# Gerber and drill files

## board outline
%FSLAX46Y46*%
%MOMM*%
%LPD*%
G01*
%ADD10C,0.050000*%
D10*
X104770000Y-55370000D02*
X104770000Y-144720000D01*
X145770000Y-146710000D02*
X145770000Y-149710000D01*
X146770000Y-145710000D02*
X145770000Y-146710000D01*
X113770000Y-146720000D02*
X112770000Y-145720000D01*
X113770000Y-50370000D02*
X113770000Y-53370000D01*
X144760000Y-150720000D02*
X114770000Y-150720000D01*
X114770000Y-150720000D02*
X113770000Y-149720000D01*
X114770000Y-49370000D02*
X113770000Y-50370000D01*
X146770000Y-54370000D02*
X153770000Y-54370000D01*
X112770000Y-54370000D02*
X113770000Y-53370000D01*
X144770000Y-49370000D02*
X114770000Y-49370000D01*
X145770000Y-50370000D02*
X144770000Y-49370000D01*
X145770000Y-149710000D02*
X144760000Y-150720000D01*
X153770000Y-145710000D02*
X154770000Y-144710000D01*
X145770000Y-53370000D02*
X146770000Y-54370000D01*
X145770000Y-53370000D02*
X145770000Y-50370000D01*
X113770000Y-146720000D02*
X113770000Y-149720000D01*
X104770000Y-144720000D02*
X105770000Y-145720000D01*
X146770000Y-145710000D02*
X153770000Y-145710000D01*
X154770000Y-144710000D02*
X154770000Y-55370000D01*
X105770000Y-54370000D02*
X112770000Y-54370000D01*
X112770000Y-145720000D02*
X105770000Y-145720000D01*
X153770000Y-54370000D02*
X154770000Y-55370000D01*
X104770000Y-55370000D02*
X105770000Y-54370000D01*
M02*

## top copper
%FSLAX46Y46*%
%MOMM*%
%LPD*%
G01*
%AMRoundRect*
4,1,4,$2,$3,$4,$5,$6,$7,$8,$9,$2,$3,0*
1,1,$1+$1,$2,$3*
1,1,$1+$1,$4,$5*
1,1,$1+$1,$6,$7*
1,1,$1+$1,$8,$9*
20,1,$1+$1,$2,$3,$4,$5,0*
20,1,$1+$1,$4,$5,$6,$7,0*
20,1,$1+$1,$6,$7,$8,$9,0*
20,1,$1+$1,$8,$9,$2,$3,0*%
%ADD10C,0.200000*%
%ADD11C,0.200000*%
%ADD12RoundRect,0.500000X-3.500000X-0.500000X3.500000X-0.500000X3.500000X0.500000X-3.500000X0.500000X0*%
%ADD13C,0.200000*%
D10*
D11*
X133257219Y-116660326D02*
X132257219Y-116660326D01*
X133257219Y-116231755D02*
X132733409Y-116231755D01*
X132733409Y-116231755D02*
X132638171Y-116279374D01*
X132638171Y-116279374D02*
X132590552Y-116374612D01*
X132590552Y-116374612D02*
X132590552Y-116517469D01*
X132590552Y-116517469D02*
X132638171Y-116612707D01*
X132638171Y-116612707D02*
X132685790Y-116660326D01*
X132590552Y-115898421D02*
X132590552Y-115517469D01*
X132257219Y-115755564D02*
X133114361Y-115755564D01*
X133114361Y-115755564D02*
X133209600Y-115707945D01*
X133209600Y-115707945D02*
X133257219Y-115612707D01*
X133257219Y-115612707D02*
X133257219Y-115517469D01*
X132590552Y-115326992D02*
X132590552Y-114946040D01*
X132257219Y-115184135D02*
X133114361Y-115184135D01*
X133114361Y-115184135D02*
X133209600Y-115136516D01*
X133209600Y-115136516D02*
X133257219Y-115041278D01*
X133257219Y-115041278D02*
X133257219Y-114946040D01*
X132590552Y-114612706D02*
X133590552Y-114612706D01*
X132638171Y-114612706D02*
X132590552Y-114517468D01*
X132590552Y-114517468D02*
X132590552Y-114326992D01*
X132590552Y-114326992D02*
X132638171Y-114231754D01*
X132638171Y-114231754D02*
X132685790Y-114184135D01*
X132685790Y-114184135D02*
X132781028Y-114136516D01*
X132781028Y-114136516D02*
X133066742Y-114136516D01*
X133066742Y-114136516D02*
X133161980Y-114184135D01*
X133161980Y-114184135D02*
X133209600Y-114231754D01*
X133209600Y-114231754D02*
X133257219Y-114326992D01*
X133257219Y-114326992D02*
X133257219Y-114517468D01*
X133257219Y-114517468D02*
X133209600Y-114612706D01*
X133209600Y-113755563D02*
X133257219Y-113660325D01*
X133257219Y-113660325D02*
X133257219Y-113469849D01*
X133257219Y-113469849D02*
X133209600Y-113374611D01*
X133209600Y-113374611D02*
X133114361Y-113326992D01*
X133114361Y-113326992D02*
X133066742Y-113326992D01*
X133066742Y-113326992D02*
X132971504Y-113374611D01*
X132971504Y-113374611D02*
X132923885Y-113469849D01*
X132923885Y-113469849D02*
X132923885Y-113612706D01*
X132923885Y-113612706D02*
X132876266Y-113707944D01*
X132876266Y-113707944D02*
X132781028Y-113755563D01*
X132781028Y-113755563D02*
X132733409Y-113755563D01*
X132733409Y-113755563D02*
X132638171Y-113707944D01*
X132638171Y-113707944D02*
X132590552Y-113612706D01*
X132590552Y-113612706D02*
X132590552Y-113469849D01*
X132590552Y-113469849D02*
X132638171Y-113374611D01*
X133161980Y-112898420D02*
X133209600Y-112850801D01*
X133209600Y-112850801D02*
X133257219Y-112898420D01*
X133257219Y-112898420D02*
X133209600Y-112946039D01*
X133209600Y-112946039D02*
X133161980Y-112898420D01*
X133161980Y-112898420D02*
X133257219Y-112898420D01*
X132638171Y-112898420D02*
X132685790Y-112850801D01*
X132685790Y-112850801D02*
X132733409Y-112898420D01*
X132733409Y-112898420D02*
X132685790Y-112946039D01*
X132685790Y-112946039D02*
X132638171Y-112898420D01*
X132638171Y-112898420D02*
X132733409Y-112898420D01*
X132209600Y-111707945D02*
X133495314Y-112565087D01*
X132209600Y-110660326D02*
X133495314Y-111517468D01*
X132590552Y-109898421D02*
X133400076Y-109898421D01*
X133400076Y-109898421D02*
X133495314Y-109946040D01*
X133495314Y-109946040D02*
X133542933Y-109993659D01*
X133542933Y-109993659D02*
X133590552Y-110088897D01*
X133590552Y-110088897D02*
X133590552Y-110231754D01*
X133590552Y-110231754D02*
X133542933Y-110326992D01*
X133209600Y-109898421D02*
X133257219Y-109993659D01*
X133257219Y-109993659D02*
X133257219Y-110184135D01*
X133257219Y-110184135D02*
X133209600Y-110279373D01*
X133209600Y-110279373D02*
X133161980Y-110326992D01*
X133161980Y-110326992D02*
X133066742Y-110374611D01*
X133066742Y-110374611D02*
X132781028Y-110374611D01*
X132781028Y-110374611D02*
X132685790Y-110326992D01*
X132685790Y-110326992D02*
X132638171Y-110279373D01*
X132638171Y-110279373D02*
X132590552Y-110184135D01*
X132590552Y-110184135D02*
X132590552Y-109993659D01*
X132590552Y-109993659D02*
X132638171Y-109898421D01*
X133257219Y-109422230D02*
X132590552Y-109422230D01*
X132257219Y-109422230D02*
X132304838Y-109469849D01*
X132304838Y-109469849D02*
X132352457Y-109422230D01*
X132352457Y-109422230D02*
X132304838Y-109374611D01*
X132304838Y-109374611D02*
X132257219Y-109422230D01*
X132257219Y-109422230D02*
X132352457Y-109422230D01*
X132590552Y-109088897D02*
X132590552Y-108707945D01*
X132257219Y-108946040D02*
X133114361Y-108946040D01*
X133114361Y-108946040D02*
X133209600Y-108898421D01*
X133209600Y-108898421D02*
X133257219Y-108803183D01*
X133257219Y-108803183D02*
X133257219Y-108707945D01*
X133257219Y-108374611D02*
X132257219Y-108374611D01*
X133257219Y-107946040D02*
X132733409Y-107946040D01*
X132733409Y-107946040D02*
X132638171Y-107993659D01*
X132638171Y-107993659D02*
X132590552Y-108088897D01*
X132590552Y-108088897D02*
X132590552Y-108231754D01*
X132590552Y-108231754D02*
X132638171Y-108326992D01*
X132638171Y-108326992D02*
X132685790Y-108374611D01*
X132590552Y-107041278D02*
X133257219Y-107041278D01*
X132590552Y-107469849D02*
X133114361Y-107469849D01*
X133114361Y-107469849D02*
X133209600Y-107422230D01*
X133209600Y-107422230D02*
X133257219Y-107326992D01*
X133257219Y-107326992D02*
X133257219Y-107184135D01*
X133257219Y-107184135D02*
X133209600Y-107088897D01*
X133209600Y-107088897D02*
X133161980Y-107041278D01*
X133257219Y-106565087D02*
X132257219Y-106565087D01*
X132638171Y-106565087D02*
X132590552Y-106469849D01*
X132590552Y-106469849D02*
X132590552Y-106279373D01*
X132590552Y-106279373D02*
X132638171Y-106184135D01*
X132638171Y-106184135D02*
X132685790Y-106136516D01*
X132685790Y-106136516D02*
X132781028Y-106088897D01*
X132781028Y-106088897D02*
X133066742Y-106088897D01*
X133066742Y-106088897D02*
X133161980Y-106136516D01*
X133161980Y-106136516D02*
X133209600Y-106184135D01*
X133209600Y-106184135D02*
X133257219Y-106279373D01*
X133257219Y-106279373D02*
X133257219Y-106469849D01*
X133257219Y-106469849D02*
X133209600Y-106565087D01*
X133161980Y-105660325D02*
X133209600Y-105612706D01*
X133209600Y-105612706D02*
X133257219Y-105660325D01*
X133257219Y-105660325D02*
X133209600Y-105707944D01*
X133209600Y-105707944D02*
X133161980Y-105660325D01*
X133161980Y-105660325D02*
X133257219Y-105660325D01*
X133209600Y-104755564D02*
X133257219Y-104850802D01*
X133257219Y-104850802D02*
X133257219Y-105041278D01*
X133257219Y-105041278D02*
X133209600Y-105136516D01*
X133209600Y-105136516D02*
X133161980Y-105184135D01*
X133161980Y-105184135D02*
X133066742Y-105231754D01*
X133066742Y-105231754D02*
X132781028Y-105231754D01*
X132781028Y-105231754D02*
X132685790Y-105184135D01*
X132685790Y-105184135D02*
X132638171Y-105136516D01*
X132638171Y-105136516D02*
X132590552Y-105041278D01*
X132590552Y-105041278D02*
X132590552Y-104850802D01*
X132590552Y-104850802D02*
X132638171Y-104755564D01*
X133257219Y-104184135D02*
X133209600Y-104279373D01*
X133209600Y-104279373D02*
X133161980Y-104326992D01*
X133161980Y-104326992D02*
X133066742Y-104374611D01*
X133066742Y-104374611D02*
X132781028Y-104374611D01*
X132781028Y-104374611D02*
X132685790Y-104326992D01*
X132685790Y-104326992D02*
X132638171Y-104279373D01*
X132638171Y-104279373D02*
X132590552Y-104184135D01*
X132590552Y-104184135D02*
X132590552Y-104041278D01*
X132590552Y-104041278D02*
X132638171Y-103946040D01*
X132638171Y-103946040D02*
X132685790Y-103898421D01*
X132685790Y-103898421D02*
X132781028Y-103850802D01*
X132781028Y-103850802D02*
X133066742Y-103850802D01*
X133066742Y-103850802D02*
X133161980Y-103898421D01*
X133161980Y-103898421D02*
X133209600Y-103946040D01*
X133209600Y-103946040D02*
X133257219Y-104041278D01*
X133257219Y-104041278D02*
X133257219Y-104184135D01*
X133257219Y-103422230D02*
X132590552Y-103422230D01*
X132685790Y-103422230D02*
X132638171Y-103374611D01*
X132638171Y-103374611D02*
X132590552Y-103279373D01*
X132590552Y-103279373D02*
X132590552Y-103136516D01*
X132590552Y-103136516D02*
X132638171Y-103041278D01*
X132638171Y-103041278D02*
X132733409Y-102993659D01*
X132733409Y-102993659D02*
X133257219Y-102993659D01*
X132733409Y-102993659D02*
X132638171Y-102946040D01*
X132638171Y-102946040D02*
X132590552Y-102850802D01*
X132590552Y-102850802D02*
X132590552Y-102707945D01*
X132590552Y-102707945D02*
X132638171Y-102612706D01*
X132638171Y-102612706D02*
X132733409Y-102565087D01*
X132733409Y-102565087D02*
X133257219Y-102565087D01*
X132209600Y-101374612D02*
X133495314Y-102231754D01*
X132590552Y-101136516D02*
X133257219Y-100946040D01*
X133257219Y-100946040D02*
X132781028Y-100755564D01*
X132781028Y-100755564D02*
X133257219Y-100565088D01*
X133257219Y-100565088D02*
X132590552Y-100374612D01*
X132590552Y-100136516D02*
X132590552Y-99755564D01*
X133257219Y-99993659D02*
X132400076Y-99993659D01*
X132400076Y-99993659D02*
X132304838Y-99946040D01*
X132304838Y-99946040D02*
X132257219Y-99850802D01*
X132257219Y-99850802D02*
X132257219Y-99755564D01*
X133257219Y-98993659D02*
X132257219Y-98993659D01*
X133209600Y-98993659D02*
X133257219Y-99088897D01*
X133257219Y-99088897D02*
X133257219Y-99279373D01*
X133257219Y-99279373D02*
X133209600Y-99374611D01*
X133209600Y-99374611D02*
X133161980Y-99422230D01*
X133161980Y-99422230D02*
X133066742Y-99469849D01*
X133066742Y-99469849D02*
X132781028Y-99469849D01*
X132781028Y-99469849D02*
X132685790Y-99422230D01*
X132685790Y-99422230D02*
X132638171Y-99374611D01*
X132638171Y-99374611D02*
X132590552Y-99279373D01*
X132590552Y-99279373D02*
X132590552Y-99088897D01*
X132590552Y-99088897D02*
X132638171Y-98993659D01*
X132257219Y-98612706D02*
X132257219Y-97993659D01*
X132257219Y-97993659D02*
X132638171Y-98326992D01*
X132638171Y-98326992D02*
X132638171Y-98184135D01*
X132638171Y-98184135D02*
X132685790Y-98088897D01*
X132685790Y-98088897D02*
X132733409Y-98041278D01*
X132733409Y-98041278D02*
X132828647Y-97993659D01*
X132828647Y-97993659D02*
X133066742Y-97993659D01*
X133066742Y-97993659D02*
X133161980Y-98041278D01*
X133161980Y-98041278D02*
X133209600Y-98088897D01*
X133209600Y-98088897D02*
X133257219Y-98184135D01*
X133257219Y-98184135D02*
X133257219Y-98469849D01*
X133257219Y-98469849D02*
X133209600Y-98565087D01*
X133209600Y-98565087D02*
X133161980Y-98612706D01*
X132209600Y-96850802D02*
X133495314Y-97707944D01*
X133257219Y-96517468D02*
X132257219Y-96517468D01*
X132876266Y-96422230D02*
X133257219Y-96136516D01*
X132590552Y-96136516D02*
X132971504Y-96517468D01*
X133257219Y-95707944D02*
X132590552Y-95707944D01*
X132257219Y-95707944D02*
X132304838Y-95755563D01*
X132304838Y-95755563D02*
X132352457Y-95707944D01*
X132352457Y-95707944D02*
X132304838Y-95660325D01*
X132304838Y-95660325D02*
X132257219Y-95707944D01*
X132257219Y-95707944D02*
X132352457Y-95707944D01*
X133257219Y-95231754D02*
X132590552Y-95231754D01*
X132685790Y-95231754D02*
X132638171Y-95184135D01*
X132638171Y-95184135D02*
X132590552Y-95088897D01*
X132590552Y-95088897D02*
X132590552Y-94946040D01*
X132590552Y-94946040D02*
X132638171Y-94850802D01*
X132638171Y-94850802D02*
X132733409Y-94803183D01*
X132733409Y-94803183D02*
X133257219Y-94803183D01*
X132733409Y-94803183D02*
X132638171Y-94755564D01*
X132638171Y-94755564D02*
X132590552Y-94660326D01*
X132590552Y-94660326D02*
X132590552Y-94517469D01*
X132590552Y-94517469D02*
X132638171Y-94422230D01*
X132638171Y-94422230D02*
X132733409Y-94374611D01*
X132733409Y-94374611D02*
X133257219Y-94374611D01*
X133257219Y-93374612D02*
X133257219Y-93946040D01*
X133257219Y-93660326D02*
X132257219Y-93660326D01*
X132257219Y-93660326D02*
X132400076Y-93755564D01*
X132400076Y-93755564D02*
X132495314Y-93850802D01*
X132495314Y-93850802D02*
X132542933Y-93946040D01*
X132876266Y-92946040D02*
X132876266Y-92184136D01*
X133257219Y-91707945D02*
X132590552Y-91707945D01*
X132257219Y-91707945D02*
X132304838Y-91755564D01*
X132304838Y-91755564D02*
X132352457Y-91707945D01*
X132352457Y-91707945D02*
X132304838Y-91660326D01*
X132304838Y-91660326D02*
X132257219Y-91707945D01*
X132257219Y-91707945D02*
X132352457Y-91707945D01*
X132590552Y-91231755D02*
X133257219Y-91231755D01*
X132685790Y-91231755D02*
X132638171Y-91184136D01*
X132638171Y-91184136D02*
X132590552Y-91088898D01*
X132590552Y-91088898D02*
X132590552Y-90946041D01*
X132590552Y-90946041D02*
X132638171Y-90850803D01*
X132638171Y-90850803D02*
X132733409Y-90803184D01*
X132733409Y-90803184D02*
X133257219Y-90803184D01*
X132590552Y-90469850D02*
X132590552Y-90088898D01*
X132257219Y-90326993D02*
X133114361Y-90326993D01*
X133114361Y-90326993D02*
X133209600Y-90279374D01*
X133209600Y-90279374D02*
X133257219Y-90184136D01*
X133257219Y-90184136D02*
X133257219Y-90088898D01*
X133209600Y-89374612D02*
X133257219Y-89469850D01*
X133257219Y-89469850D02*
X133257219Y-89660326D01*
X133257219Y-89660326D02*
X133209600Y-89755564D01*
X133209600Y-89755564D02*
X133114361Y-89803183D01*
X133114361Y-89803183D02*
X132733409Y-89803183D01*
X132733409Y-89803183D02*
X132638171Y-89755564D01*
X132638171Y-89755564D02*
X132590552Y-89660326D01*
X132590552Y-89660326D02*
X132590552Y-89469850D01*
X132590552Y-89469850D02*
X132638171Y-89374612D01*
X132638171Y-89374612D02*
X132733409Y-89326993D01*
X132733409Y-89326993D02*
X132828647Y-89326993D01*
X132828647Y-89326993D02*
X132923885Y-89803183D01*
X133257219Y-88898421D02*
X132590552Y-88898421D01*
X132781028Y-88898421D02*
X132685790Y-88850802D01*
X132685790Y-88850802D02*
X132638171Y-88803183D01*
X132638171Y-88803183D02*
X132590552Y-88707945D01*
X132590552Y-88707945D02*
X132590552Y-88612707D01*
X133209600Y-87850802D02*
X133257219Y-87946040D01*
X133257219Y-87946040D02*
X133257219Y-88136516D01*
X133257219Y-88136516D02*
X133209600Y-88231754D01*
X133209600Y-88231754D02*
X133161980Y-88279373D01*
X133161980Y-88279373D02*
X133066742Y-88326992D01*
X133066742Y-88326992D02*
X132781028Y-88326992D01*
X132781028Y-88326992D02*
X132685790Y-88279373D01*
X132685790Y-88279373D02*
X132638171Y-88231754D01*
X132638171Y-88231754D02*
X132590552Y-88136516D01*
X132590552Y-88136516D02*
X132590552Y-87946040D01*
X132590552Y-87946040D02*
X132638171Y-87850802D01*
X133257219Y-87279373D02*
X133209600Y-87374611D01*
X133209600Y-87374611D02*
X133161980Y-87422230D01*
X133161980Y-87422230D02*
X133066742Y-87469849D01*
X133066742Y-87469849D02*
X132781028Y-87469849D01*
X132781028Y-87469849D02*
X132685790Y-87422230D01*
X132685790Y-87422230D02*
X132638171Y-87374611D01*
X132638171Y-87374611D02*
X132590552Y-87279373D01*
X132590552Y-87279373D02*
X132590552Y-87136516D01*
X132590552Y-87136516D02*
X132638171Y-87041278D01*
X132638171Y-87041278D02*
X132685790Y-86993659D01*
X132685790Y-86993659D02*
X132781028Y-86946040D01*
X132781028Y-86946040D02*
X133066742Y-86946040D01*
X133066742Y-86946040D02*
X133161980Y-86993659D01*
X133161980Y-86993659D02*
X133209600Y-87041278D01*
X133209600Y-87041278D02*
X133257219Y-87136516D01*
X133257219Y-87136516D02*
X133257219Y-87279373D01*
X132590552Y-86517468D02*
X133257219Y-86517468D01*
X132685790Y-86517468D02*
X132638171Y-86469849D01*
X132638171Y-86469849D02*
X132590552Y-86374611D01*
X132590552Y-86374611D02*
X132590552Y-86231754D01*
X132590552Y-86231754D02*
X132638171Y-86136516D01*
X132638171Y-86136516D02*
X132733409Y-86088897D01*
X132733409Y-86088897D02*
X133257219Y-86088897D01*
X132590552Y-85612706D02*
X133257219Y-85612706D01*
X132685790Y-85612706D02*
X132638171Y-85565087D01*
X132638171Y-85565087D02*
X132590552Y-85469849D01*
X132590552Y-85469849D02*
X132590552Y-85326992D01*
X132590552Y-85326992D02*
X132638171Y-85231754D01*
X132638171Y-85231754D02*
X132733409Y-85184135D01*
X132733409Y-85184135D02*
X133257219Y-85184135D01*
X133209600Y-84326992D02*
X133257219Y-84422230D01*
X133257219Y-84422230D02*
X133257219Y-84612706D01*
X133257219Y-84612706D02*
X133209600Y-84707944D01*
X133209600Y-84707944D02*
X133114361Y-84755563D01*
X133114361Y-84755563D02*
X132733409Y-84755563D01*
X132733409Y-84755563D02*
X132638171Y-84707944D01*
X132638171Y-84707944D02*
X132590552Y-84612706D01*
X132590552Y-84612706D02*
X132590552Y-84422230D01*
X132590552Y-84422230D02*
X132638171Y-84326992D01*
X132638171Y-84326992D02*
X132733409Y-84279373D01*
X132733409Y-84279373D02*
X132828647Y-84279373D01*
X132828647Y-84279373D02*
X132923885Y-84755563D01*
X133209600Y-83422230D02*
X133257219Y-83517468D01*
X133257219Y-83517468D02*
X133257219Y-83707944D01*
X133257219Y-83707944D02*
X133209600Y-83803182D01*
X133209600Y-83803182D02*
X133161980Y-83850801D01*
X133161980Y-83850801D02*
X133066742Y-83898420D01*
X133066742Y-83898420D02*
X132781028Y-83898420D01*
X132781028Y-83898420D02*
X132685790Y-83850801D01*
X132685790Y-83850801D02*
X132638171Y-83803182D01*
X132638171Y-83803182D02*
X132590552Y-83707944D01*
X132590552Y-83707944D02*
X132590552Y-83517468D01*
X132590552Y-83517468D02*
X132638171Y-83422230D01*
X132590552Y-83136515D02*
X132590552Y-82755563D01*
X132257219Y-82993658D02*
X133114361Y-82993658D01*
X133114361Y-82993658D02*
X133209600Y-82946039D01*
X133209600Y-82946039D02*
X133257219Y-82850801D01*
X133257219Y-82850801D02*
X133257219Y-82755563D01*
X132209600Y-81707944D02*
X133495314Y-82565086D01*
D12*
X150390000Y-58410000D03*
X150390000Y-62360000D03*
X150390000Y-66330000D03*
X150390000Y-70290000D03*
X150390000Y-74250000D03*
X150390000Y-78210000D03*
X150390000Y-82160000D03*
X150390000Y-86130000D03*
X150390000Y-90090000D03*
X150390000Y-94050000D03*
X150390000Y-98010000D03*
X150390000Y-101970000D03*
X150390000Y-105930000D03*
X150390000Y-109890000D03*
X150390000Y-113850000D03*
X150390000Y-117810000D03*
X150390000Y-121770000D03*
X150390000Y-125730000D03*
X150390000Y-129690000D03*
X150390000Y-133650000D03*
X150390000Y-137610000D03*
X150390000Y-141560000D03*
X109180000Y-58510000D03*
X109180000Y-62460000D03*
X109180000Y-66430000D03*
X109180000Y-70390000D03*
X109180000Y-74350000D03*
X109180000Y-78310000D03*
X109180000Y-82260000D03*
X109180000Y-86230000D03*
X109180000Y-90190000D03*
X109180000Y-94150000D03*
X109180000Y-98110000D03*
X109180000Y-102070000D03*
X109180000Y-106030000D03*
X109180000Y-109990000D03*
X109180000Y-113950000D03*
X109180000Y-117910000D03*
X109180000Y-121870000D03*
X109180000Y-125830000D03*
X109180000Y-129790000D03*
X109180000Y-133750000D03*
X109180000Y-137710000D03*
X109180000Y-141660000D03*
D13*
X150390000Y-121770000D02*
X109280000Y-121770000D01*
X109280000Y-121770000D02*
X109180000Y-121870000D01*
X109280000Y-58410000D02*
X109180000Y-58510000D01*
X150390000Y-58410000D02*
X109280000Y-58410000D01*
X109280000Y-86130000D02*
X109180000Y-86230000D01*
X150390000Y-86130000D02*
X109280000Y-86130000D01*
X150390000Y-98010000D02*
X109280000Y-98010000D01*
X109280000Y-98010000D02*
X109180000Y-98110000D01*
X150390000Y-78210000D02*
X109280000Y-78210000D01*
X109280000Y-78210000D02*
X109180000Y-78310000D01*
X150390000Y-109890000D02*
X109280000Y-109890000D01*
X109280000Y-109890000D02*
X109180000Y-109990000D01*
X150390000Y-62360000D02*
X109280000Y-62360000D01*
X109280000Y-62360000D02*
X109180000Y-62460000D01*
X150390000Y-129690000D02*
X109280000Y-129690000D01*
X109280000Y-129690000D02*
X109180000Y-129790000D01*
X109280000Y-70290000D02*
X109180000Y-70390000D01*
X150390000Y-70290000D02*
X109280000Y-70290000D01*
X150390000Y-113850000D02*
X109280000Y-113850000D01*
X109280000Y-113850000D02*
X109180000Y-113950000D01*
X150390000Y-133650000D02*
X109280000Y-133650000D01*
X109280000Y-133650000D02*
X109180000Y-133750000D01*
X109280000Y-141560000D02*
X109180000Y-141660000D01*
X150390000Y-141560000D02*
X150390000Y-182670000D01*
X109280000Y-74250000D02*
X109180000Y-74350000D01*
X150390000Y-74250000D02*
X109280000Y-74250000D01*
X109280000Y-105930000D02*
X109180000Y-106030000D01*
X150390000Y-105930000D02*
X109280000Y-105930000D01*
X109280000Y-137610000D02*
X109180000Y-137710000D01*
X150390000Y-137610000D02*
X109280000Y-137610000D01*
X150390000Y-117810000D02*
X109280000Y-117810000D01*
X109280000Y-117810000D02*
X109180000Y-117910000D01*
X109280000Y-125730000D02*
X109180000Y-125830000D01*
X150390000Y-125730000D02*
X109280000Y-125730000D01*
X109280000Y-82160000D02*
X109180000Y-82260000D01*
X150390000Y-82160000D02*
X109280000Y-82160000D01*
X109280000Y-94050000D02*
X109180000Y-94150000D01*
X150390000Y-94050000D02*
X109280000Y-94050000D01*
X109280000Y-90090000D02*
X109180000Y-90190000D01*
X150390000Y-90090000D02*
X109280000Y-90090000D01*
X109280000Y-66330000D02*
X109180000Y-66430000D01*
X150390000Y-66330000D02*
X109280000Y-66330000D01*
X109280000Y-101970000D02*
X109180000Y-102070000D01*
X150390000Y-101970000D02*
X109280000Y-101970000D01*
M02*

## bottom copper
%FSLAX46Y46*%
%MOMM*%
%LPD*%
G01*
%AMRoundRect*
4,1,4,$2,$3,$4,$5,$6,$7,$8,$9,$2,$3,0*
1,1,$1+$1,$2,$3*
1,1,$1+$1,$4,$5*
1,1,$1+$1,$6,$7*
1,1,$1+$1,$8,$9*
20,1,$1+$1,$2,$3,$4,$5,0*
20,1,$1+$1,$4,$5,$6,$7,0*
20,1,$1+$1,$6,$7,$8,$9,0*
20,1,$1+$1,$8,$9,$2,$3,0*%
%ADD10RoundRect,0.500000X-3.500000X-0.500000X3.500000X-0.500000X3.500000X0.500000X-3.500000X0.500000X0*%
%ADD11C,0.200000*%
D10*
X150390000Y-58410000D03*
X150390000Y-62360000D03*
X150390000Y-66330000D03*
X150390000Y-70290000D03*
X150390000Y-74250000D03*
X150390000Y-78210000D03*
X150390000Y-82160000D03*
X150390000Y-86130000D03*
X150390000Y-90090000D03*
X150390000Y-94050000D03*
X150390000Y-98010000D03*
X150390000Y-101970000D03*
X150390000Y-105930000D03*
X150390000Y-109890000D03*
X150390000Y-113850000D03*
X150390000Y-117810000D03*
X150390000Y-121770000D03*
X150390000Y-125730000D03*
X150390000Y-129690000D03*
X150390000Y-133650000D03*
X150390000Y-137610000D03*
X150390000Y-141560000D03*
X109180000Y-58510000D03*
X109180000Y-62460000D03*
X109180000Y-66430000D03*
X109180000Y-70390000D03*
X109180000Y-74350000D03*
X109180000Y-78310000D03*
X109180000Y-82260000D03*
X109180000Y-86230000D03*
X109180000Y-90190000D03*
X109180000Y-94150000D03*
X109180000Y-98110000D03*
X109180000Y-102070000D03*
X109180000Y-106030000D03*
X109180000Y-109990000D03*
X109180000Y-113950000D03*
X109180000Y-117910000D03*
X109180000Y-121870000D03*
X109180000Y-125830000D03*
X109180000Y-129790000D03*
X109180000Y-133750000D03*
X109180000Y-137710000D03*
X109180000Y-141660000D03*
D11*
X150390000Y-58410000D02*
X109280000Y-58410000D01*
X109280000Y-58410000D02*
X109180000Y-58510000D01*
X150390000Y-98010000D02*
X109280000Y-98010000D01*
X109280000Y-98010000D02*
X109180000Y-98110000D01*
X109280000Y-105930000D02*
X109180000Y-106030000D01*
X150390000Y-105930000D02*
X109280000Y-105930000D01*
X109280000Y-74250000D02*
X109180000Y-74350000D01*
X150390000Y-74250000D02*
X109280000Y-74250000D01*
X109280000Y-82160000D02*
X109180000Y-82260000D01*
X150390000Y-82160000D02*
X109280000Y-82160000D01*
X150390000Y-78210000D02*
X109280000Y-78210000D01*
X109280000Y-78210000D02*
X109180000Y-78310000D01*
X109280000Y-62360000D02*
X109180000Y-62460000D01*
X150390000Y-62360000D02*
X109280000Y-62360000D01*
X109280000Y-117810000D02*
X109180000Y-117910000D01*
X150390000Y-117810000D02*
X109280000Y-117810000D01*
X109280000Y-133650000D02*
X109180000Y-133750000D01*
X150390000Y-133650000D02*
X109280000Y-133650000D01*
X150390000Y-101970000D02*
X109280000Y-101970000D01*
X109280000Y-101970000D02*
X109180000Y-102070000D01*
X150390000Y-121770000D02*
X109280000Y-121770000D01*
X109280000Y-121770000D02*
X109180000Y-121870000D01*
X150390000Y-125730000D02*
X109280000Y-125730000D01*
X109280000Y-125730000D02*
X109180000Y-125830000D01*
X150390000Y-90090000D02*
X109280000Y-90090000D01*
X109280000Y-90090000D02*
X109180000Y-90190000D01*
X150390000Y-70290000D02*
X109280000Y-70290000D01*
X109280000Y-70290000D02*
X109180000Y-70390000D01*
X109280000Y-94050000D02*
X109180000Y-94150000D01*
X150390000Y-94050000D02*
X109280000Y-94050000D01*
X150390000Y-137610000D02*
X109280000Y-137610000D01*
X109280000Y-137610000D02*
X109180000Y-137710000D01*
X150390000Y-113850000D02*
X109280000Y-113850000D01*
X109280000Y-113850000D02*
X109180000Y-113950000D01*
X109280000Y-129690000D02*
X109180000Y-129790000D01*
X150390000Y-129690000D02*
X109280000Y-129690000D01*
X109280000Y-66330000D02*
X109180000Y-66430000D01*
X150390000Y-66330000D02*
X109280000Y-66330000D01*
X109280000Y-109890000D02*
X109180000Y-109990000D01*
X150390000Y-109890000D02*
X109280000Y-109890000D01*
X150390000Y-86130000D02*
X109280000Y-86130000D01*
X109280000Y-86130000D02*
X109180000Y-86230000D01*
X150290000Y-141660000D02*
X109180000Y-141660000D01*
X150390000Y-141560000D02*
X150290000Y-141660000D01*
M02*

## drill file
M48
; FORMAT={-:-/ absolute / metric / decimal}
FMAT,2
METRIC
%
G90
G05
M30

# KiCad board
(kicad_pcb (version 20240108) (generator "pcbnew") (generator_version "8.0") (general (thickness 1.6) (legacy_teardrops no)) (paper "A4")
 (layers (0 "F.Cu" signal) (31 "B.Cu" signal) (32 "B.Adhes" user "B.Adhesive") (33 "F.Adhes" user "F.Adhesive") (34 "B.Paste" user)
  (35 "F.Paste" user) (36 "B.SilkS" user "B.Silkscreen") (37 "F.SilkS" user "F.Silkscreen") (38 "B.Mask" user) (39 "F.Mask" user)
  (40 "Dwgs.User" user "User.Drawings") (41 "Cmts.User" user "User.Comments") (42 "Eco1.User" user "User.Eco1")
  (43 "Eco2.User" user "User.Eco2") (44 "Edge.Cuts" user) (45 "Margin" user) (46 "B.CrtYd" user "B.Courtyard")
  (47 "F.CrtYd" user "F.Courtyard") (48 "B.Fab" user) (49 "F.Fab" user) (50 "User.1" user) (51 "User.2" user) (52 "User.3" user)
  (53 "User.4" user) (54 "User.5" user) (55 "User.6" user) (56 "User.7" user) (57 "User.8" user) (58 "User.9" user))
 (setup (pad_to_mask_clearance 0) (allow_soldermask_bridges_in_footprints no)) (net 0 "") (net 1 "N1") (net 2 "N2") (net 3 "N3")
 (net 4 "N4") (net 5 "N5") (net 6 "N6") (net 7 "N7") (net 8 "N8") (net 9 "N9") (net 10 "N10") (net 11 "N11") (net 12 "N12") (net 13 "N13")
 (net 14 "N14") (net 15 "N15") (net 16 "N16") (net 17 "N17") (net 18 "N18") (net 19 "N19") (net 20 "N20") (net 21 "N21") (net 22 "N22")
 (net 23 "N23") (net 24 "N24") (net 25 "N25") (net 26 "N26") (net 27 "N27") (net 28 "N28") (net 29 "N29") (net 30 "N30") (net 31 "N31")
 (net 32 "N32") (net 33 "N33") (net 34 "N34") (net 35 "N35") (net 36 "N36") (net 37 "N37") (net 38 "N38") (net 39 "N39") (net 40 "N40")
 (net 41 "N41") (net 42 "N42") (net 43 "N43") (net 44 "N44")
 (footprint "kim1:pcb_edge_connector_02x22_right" (layer "F.Cu") (at 145.04 98.96)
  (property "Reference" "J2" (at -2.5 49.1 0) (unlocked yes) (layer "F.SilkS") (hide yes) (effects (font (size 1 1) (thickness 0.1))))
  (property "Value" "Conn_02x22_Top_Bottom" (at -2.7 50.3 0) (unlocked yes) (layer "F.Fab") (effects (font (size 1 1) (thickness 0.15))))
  (pad "1" connect roundrect (at 5.35 -40.55) (size 8 2) (layers "F.Cu" "F.Mask") (roundrect_rratio 0.25) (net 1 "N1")
   (thermal_bridge_angle 45))
  (pad "2" connect roundrect (at 5.35 -36.6) (size 8 2) (layers "F.Cu" "F.Mask") (roundrect_rratio 0.25) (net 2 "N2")
   (thermal_bridge_angle 45))
  (pad "3" connect roundrect (at 5.35 -32.63) (size 8 2) (layers "F.Cu" "F.Mask") (roundrect_rratio 0.25) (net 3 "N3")
   (thermal_bridge_angle 45))
  (pad "4" connect roundrect (at 5.35 -28.67) (size 8 2) (layers "F.Cu" "F.Mask") (roundrect_rratio 0.25) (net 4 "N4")
   (thermal_bridge_angle 45))
  (pad "5" connect roundrect (at 5.35 -24.71) (size 8 2) (layers "F.Cu" "F.Mask") (roundrect_rratio 0.25) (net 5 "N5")
   (thermal_bridge_angle 45))
  (pad "6" connect roundrect (at 5.35 -20.75) (size 8 2) (layers "F.Cu" "F.Mask") (roundrect_rratio 0.25) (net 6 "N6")
   (thermal_bridge_angle 45))
  (pad "7" connect roundrect (at 5.35 -16.8) (size 8 2) (layers "F.Cu" "F.Mask") (roundrect_rratio 0.25) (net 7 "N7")
   (thermal_bridge_angle 45))
  (pad "8" connect roundrect (at 5.35 -12.83) (size 8 2) (layers "F.Cu" "F.Mask") (roundrect_rratio 0.25) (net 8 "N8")
   (thermal_bridge_angle 45))
  (pad "9" connect roundrect (at 5.35 -8.87) (size 8 2) (layers "F.Cu" "F.Mask") (roundrect_rratio 0.25) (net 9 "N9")
   (thermal_bridge_angle 45))
  (pad "10" connect roundrect (at 5.35 -4.91) (size 8 2) (layers "F.Cu" "F.Mask") (roundrect_rratio 0.25) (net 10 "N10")
   (thermal_bridge_angle 45))
  (pad "11" connect roundrect (at 5.35 -0.95) (size 8 2) (layers "F.Cu" "F.Mask") (roundrect_rratio 0.25) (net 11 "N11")
   (thermal_bridge_angle 45))
  (pad "12" connect roundrect (at 5.35 3.01) (size 8 2) (layers "F.Cu" "F.Mask") (roundrect_rratio 0.25) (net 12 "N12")
   (thermal_bridge_angle 45))
  (pad "13" connect roundrect (at 5.35 6.97) (size 8 2) (layers "F.Cu" "F.Mask") (roundrect_rratio 0.25) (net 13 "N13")
   (thermal_bridge_angle 45))
  (pad "14" connect roundrect (at 5.35 10.93) (size 8 2) (layers "F.Cu" "F.Mask") (roundrect_rratio 0.25) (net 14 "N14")
   (thermal_bridge_angle 45))
  (pad "15" connect roundrect (at 5.35 14.89) (size 8 2) (layers "F.Cu" "F.Mask") (roundrect_rratio 0.25) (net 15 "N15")
   (thermal_bridge_angle 45))
  (pad "16" connect roundrect (at 5.35 18.85) (size 8 2) (layers "F.Cu" "F.Mask") (roundrect_rratio 0.25) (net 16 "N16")
   (thermal_bridge_angle 45))
  (pad "17" connect roundrect (at 5.35 22.81) (size 8 2) (layers "F.Cu" "F.Mask") (roundrect_rratio 0.25) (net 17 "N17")
   (thermal_bridge_angle 45))
  (pad "18" connect roundrect (at 5.35 26.77) (size 8 2) (layers "F.Cu" "F.Mask") (roundrect_rratio 0.25) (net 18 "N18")
   (thermal_bridge_angle 45))
  (pad "19" connect roundrect (at 5.35 30.73) (size 8 2) (layers "F.Cu" "F.Mask") (roundrect_rratio 0.25) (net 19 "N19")
   (thermal_bridge_angle 45))
  (pad "20" connect roundrect (at 5.35 34.69) (size 8 2) (layers "F.Cu" "F.Mask") (roundrect_rratio 0.25) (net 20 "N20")
   (thermal_bridge_angle 45))
  (pad "21" connect roundrect (at 5.35 38.65) (size 8 2) (layers "F.Cu" "F.Mask") (roundrect_rratio 0.25) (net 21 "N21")
   (thermal_bridge_angle 45))
  (pad "22" connect roundrect (at 5.35 42.6) (size 8 2) (layers "F.Cu" "F.Mask") (roundrect_rratio 0.25) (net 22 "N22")
   (thermal_bridge_angle 45))
  (pad "A" connect roundrect (at 5.35 -40.55) (size 8 2) (layers "B.Cu" "B.SilkS" "F.Mask") (roundrect_rratio 0.25) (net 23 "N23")
   (thermal_bridge_angle 45))
  (pad "B" connect roundrect (at 5.35 -36.6) (size 8 2) (layers "B.Cu" "F.Mask") (roundrect_rratio 0.25) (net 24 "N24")
   (thermal_bridge_angle 45))
  (pad "C" connect roundrect (at 5.35 -32.63) (size 8 2) (layers "B.Cu" "F.Mask") (roundrect_rratio 0.25) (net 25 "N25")
   (thermal_bridge_angle 45))
  (pad "D" connect roundrect (at 5.35 -28.67) (size 8 2) (layers "B.Cu" "F.Mask") (roundrect_rratio 0.25) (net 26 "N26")
   (thermal_bridge_angle 45))
  (pad "E" connect roundrect (at 5.35 -24.71) (size 8 2) (layers "B.Cu" "F.Mask") (roundrect_rratio 0.25) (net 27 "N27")
   (thermal_bridge_angle 45))
  (pad "F" connect roundrect (at 5.35 -20.75) (size 8 2) (layers "B.Cu" "F.Mask") (roundrect_rratio 0.25) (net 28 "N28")
   (thermal_bridge_angle 45))
  (pad "H" connect roundrect (at 5.35 -16.8) (size 8 2) (layers "B.Cu" "F.Mask") (roundrect_rratio 0.25) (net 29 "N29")
   (thermal_bridge_angle 45))
  (pad "J" connect roundrect (at 5.35 -12.83) (size 8 2) (layers "B.Cu" "F.Mask") (roundrect_rratio 0.25) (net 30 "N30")
   (thermal_bridge_angle 45))
  (pad "K" connect roundrect (at 5.35 -8.87) (size 8 2) (layers "B.Cu" "F.Mask") (roundrect_rratio 0.25) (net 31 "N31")
   (thermal_bridge_angle 45))
  (pad "L" connect roundrect (at 5.35 -4.91) (size 8 2) (layers "B.Cu" "F.Mask") (roundrect_rratio 0.25) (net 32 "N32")
   (thermal_bridge_angle 45))
  (pad "M" connect roundrect (at 5.35 -0.95) (size 8 2) (layers "B.Cu" "F.Mask") (roundrect_rratio 0.25) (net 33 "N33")
   (thermal_bridge_angle 45))
  (pad "N" connect roundrect (at 5.35 3.01) (size 8 2) (layers "B.Cu" "F.Mask") (roundrect_rratio 0.25) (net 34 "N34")
   (thermal_bridge_angle 45))
  (pad "P" connect roundrect (at 5.35 6.97) (size 8 2) (layers "B.Cu" "F.Mask") (roundrect_rratio 0.25) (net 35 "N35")
   (thermal_bridge_angle 45))
  (pad "R" connect roundrect (at 5.35 10.93) (size 8 2) (layers "B.Cu" "F.Mask") (roundrect_rratio 0.25) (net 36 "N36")
   (thermal_bridge_angle 45))
  (pad "S" connect roundrect (at 5.35 14.89) (size 8 2) (layers "B.Cu" "F.Mask") (roundrect_rratio 0.25) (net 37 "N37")
   (thermal_bridge_angle 45))
  (pad "T" connect roundrect (at 5.35 18.85) (size 8 2) (layers "B.Cu" "F.Mask") (roundrect_rratio 0.25) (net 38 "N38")
   (thermal_bridge_angle 45))
  (pad "U" connect roundrect (at 5.35 22.81) (size 8 2) (layers "B.Cu" "F.Mask") (roundrect_rratio 0.25) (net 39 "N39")
   (thermal_bridge_angle 45))
  (pad "V" connect roundrect (at 5.35 26.77) (size 8 2) (layers "B.Cu" "F.Mask") (roundrect_rratio 0.25) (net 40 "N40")
   (thermal_bridge_angle 45))
  (pad "W" connect roundrect (at 5.35 30.73) (size 8 2) (layers "B.Cu" "F.Mask") (roundrect_rratio 0.25) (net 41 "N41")
   (thermal_bridge_angle 45))
  (pad "X" connect roundrect (at 5.35 34.69) (size 8 2) (layers "B.Cu" "F.Mask") (roundrect_rratio 0.25) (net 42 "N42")
   (thermal_bridge_angle 45))
  (pad "Y" connect roundrect (at 5.35 38.65) (size 8 2) (layers "B.Cu" "F.Mask") (roundrect_rratio 0.25) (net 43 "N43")
   (thermal_bridge_angle 45))
  (pad "Z" connect roundrect (at 5.35 42.6) (size 8 2) (layers "B.Cu" "F.Mask") (roundrect_rratio 0.25) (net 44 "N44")
   (thermal_bridge_angle 45)))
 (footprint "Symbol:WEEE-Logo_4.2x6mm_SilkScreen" (layer "F.Cu") (at 129.71 141.81 90)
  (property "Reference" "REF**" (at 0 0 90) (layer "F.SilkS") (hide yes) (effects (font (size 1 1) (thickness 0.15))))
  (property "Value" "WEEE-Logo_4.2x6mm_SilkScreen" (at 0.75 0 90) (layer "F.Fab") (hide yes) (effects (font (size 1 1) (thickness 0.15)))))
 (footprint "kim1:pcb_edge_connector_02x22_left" (layer "F.Cu") (at 111.83 99.06)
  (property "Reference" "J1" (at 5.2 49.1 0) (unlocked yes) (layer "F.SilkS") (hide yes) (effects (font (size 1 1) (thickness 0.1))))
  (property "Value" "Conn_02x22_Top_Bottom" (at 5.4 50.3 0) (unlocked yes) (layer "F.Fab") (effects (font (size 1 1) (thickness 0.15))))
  (pad "1" connect roundrect (at -2.65 -40.55) (size 8 2) (layers "F.Cu" "F.Mask") (roundrect_rratio 0.25) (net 1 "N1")
   (thermal_bridge_angle 45))
  (pad "2" connect roundrect (at -2.65 -36.6) (size 8 2) (layers "F.Cu" "F.Mask") (roundrect_rratio 0.25) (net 2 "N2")
   (thermal_bridge_angle 45))
  (pad "3" connect roundrect (at -2.65 -32.63) (size 8 2) (layers "F.Cu" "F.Mask") (roundrect_rratio 0.25) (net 3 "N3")
   (thermal_bridge_angle 45))
  (pad "4" connect roundrect (at -2.65 -28.67) (size 8 2) (layers "F.Cu" "F.Mask") (roundrect_rratio 0.25) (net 4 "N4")
   (thermal_bridge_angle 45))
  (pad "5" connect roundrect (at -2.65 -24.71) (size 8 2) (layers "F.Cu" "F.Mask") (roundrect_rratio 0.25) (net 5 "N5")
   (thermal_bridge_angle 45))
  (pad "6" connect roundrect (at -2.65 -20.75) (size 8 2) (layers "F.Cu" "F.Mask") (roundrect_rratio 0.25) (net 6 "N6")
   (thermal_bridge_angle 45))
  (pad "7" connect roundrect (at -2.65 -16.8) (size 8 2) (layers "F.Cu" "F.Mask") (roundrect_rratio 0.25) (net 7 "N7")
   (thermal_bridge_angle 45))
  (pad "8" connect roundrect (at -2.65 -12.83) (size 8 2) (layers "F.Cu" "F.Mask") (roundrect_rratio 0.25) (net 8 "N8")
   (thermal_bridge_angle 45))
  (pad "9" connect roundrect (at -2.65 -8.87) (size 8 2) (layers "F.Cu" "F.Mask") (roundrect_rratio 0.25) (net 9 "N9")
   (thermal_bridge_angle 45))
  (pad "10" connect roundrect (at -2.65 -4.91) (size 8 2) (layers "F.Cu" "F.Mask") (roundrect_rratio 0.25) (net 10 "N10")
   (thermal_bridge_angle 45))
  (pad "11" connect roundrect (at -2.65 -0.95) (size 8 2) (layers "F.Cu" "F.Mask") (roundrect_rratio 0.25) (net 11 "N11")
   (thermal_bridge_angle 45))
  (pad "12" connect roundrect (at -2.65 3.01) (size 8 2) (layers "F.Cu" "F.Mask") (roundrect_rratio 0.25) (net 12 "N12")
   (thermal_bridge_angle 45))
  (pad "13" connect roundrect (at -2.65 6.97) (size 8 2) (layers "F.Cu" "F.Mask") (roundrect_rratio 0.25) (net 13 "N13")
   (thermal_bridge_angle 45))
  (pad "14" connect roundrect (at -2.65 10.93) (size 8 2) (layers "F.Cu" "F.Mask") (roundrect_rratio 0.25) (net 14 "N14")
   (thermal_bridge_angle 45))
  (pad "15" connect roundrect (at -2.65 14.89) (size 8 2) (layers "F.Cu" "F.Mask") (roundrect_rratio 0.25) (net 15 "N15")
   (thermal_bridge_angle 45))
  (pad "16" connect roundrect (at -2.65 18.85) (size 8 2) (layers "F.Cu" "F.Mask") (roundrect_rratio 0.25) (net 16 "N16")
   (thermal_bridge_angle 45))
  (pad "17" connect roundrect (at -2.65 22.81) (size 8 2) (layers "F.Cu" "F.Mask") (roundrect_rratio 0.25) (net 17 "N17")
   (thermal_bridge_angle 45))
  (pad "18" connect roundrect (at -2.65 26.77) (size 8 2) (layers "F.Cu" "F.Mask") (roundrect_rratio 0.25) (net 18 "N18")
   (thermal_bridge_angle 45))
  (pad "19" connect roundrect (at -2.65 30.73) (size 8 2) (layers "F.Cu" "F.Mask") (roundrect_rratio 0.25) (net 19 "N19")
   (thermal_bridge_angle 45))
  (pad "20" connect roundrect (at -2.65 34.69) (size 8 2) (layers "F.Cu" "F.Mask") (roundrect_rratio 0.25) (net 20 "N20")
   (thermal_bridge_angle 45))
  (pad "21" connect roundrect (at -2.65 38.65) (size 8 2) (layers "F.Cu" "F.Mask") (roundrect_rratio 0.25) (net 21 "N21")
   (thermal_bridge_angle 45))
  (pad "22" connect roundrect (at -2.65 42.6) (size 8 2) (layers "F.Cu" "F.Mask") (roundrect_rratio 0.25) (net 22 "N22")
   (thermal_bridge_angle 45))
  (pad "A" connect roundrect (at -2.65 -40.55) (size 8 2) (layers "B.Cu" "B.SilkS" "F.Mask") (roundrect_rratio 0.25) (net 23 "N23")
   (thermal_bridge_angle 45))
  (pad "B" connect roundrect (at -2.65 -36.6) (size 8 2) (layers "B.Cu" "F.Mask") (roundrect_rratio 0.25) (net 24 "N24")
   (thermal_bridge_angle 45))
  (pad "C" connect roundrect (at -2.65 -32.63) (size 8 2) (layers "B.Cu" "F.Mask") (roundrect_rratio 0.25) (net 25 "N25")
   (thermal_bridge_angle 45))
  (pad "D" connect roundrect (at -2.65 -28.67) (size 8 2) (layers "B.Cu" "F.Mask") (roundrect_rratio 0.25) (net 26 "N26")
   (thermal_bridge_angle 45))
  (pad "E" connect roundrect (at -2.65 -24.71) (size 8 2) (layers "B.Cu" "F.Mask") (roundrect_rratio 0.25) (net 27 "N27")
   (thermal_bridge_angle 45))
  (pad "F" connect roundrect (at -2.65 -20.75) (size 8 2) (layers "B.Cu" "F.Mask") (roundrect_rratio 0.25) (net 28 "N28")
   (thermal_bridge_angle 45))
  (pad "H" connect roundrect (at -2.65 -16.8) (size 8 2) (layers "B.Cu" "F.Mask") (roundrect_rratio 0.25) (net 29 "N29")
   (thermal_bridge_angle 45))
  (pad "J" connect roundrect (at -2.65 -12.83) (size 8 2) (layers "B.Cu" "F.Mask") (roundrect_rratio 0.25) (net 30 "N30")
   (thermal_bridge_angle 45))
  (pad "K" connect roundrect (at -2.65 -8.87) (size 8 2) (layers "B.Cu" "F.Mask") (roundrect_rratio 0.25) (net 31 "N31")
   (thermal_bridge_angle 45))
  (pad "L" connect roundrect (at -2.65 -4.91) (size 8 2) (layers "B.Cu" "F.Mask") (roundrect_rratio 0.25) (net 32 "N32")
   (thermal_bridge_angle 45))
  (pad "M" connect roundrect (at -2.65 -0.95) (size 8 2) (layers "B.Cu" "F.Mask") (roundrect_rratio 0.25) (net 33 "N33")
   (thermal_bridge_angle 45))
  (pad "N" connect roundrect (at -2.65 3.01) (size 8 2) (layers "B.Cu" "F.Mask") (roundrect_rratio 0.25) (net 34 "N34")
   (thermal_bridge_angle 45))
  (pad "P" connect roundrect (at -2.65 6.97) (size 8 2) (layers "B.Cu" "F.Mask") (roundrect_rratio 0.25) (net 35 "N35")
   (thermal_bridge_angle 45))
  (pad "R" connect roundrect (at -2.65 10.93) (size 8 2) (layers "B.Cu" "F.Mask") (roundrect_rratio 0.25) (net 36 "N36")
   (thermal_bridge_angle 45))
  (pad "S" connect roundrect (at -2.65 14.89) (size 8 2) (layers "B.Cu" "F.Mask") (roundrect_rratio 0.25) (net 37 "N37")
   (thermal_bridge_angle 45))
  (pad "T" connect roundrect (at -2.65 18.85) (size 8 2) (layers "B.Cu" "F.Mask") (roundrect_rratio 0.25) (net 38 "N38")
   (thermal_bridge_angle 45))
  (pad "U" connect roundrect (at -2.65 22.81) (size 8 2) (layers "B.Cu" "F.Mask") (roundrect_rratio 0.25) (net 39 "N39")
   (thermal_bridge_angle 45))
  (pad "V" connect roundrect (at -2.65 26.77) (size 8 2) (layers "B.Cu" "F.Mask") (roundrect_rratio 0.25) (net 40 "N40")
   (thermal_bridge_angle 45))
  (pad "W" connect roundrect (at -2.65 30.73) (size 8 2) (layers "B.Cu" "F.Mask") (roundrect_rratio 0.25) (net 41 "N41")
   (thermal_bridge_angle 45))
  (pad "X" connect roundrect (at -2.65 34.69) (size 8 2) (layers "B.Cu" "F.Mask") (roundrect_rratio 0.25) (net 42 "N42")
   (thermal_bridge_angle 45))
  (pad "Y" connect roundrect (at -2.65 38.65) (size 8 2) (layers "B.Cu" "F.Mask") (roundrect_rratio 0.25) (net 43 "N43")
   (thermal_bridge_angle 45))
  (pad "Z" connect roundrect (at -2.65 42.6) (size 8 2) (layers "B.Cu" "F.Mask") (roundrect_rratio 0.25) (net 44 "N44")
   (thermal_bridge_angle 45)))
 (gr_line (start 104.77 55.37) (end 104.77 144.72) (stroke (width 0.05) (type default)) (layer "Edge.Cuts"))
 (gr_line (start 145.77 146.71) (end 145.77 149.71) (stroke (width 0.05) (type default)) (layer "Edge.Cuts"))
 (gr_line (start 146.77 145.71) (end 145.77 146.71) (stroke (width 0.05) (type default)) (layer "Edge.Cuts"))
 (gr_line (start 113.77 146.72) (end 112.77 145.72) (stroke (width 0.05) (type default)) (layer "Edge.Cuts"))
 (gr_line (start 113.77 50.37) (end 113.77 53.37) (stroke (width 0.05) (type default)) (layer "Edge.Cuts"))
 (gr_line (start 144.76 150.72) (end 114.77 150.72) (stroke (width 0.05) (type default)) (layer "Edge.Cuts"))
 (gr_line (start 114.77 150.72) (end 113.77 149.72) (stroke (width 0.05) (type default)) (layer "Edge.Cuts"))
 (gr_line (start 114.77 49.37) (end 113.77 50.37) (stroke (width 0.05) (type default)) (layer "Edge.Cuts"))
 (gr_line (start 146.77 54.37) (end 153.77 54.37) (stroke (width 0.05) (type default)) (layer "Edge.Cuts"))
 (gr_line (start 112.77 54.37) (end 113.77 53.37) (stroke (width 0.05) (type default)) (layer "Edge.Cuts"))
 (gr_line (start 144.77 49.37) (end 114.77 49.37) (stroke (width 0.05) (type default)) (layer "Edge.Cuts"))
 (gr_line (start 145.77 50.37) (end 144.77 49.37) (stroke (width 0.05) (type default)) (layer "Edge.Cuts"))
 (gr_line (start 145.77 149.71) (end 144.76 150.72) (stroke (width 0.05) (type default)) (layer "Edge.Cuts"))
 (gr_line (start 153.77 145.71) (end 154.77 144.71) (stroke (width 0.05) (type default)) (layer "Edge.Cuts"))
 (gr_line (start 145.77 53.37) (end 146.77 54.37) (stroke (width 0.05) (type default)) (layer "Edge.Cuts"))
 (gr_line (start 145.77 53.37) (end 145.77 50.37) (stroke (width 0.05) (type default)) (layer "Edge.Cuts"))
 (gr_line (start 113.77 146.72) (end 113.77 149.72) (stroke (width 0.05) (type default)) (layer "Edge.Cuts"))
 (gr_line (start 104.77 144.72) (end 105.77 145.72) (stroke (width 0.05) (type default)) (layer "Edge.Cuts"))
 (gr_line (start 146.77 145.71) (end 153.77 145.71) (stroke (width 0.05) (type default)) (layer "Edge.Cuts"))
 (gr_line (start 154.77 144.71) (end 154.77 55.37) (stroke (width 0.05) (type default)) (layer "Edge.Cuts"))
 (gr_line (start 105.77 54.37) (end 112.77 54.37) (stroke (width 0.05) (type default)) (layer "Edge.Cuts"))
 (gr_line (start 112.77 145.72) (end 105.77 145.72) (stroke (width 0.05) (type default)) (layer "Edge.Cuts"))
 (gr_line (start 153.77 54.37) (end 154.77 55.37) (stroke (width 0.05) (type default)) (layer "Edge.Cuts"))
 (gr_line (start 104.77 55.37) (end 105.77 54.37) (stroke (width 0.05) (type default)) (layer "Edge.Cuts"))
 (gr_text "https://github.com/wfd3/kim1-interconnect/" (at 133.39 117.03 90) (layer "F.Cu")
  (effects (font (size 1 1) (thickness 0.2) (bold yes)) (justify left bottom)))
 (segment (start 150.39 58.41) (end 109.28 58.41) (width 0.2) (layer "B.Cu") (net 23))
 (segment (start 109.28 58.41) (end 109.18 58.51) (width 0.2) (layer "B.Cu") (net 23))
 (segment (start 150.39 121.77) (end 109.28 121.77) (width 0.2) (layer "F.Cu") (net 17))
 (segment (start 109.28 121.77) (end 109.18 121.87) (width 0.2) (layer "F.Cu") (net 17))
 (segment (start 109.28 58.41) (end 109.18 58.51) (width 0.2) (layer "F.Cu") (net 1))
 (segment (start 150.39 58.41) (end 109.28 58.41) (width 0.2) (layer "F.Cu") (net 1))
 (segment (start 150.39 98.01) (end 109.28 98.01) (width 0.2) (layer "B.Cu") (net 33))
 (segment (start 109.28 98.01) (end 109.18 98.11) (width 0.2) (layer "B.Cu") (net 33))
 (segment (start 109.28 86.13) (end 109.18 86.23) (width 0.2) (layer "F.Cu") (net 8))
 (segment (start 150.39 86.13) (end 109.28 86.13) (width 0.2) (layer "F.Cu") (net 8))
 (segment (start 109.28 105.93) (end 109.18 106.03) (width 0.2) (layer "B.Cu") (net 35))
 (segment (start 150.39 105.93) (end 109.28 105.93) (width 0.2) (layer "B.Cu") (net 35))
 (segment (start 109.28 74.25) (end 109.18 74.35) (width 0.2) (layer "B.Cu") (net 27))
 (segment (start 150.39 74.25) (end 109.28 74.25) (width 0.2) (layer "B.Cu") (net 27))
 (segment (start 150.39 98.01) (end 109.28 98.01) (width 0.2) (layer "F.Cu") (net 11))
 (segment (start 109.28 98.01) (end 109.18 98.11) (width 0.2) (layer "F.Cu") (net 11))
 (segment (start 109.28 82.16) (end 109.18 82.26) (width 0.2) (layer "B.Cu") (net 29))
 (segment (start 150.39 82.16) (end 109.28 82.16) (width 0.2) (layer "B.Cu") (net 29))
 (segment (start 150.39 78.21) (end 109.28 78.21) (width 0.2) (layer "F.Cu") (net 6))
 (segment (start 109.28 78.21) (end 109.18 78.31) (width 0.2) (layer "F.Cu") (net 6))
 (segment (start 150.39 109.89) (end 109.28 109.89) (width 0.2) (layer "F.Cu") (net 14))
 (segment (start 109.28 109.89) (end 109.18 109.99) (width 0.2) (layer "F.Cu") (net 14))
 (segment (start 150.39 78.21) (end 109.28 78.21) (width 0.2) (layer "B.Cu") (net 28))
 (segment (start 109.28 78.21) (end 109.18 78.31) (width 0.2) (layer "B.Cu") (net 28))
 (segment (start 109.28 62.36) (end 109.18 62.46) (width 0.2) (layer "B.Cu") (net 24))
 (segment (start 150.39 62.36) (end 109.28 62.36) (width 0.2) (layer "B.Cu") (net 24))
 (segment (start 109.28 117.81) (end 109.18 117.91) (width 0.2) (layer "B.Cu") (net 38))
 (segment (start 150.39 117.81) (end 109.28 117.81) (width 0.2) (layer "B.Cu") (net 38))
 (segment (start 150.39 62.36) (end 109.28 62.36) (width 0.2) (layer "F.Cu") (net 2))
 (segment (start 109.28 62.36) (end 109.18 62.46) (width 0.2) (layer "F.Cu") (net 2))
 (segment (start 150.39 129.69) (end 109.28 129.69) (width 0.2) (layer "F.Cu") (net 19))
 (segment (start 109.28 129.69) (end 109.18 129.79) (width 0.2) (layer "F.Cu") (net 19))
 (segment (start 109.28 70.29) (end 109.18 70.39) (width 0.2) (layer "F.Cu") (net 4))
 (segment (start 150.39 70.29) (end 109.28 70.29) (width 0.2) (layer "F.Cu") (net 4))
 (segment (start 109.28 133.65) (end 109.18 133.75) (width 0.2) (layer "B.Cu") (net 42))
 (segment (start 150.39 133.65) (end 109.28 133.65) (width 0.2) (layer "B.Cu") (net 42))
 (segment (start 150.39 113.85) (end 109.28 113.85) (width 0.2) (layer "F.Cu") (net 15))
 (segment (start 109.28 113.85) (end 109.18 113.95) (width 0.2) (layer "F.Cu") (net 15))
 (segment (start 150.39 133.65) (end 109.28 133.65) (width 0.2) (layer "F.Cu") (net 20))
 (segment (start 109.28 133.65) (end 109.18 133.75) (width 0.2) (layer "F.Cu") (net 20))
 (segment (start 150.39 101.97) (end 109.28 101.97) (width 0.2) (layer "B.Cu") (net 34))
 (segment (start 109.28 101.97) (end 109.18 102.07) (width 0.2) (layer "B.Cu") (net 34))
 (segment (start 109.28 141.56) (end 109.18 141.66) (width 0.2) (layer "F.Cu") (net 22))
 (segment (start 150.39 141.56) (end 150.39 182.67) (width 0.2) (layer "F.Cu") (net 22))
 (segment (start 150.39 121.77) (end 109.28 121.77) (width 0.2) (layer "B.Cu") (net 39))
 (segment (start 109.28 121.77) (end 109.18 121.87) (width 0.2) (layer "B.Cu") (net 39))
 (segment (start 150.39 125.73) (end 109.28 125.73) (width 0.2) (layer "B.Cu") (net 40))
 (segment (start 109.28 125.73) (end 109.18 125.83) (width 0.2) (layer "B.Cu") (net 40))
 (segment (start 109.28 74.25) (end 109.18 74.35) (width 0.2) (layer "F.Cu") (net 5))
 (segment (start 150.39 74.25) (end 109.28 74.25) (width 0.2) (layer "F.Cu") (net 5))
 (segment (start 109.28 105.93) (end 109.18 106.03) (width 0.2) (layer "F.Cu") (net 13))
 (segment (start 150.39 105.93) (end 109.28 105.93) (width 0.2) (layer "F.Cu") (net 13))
 (segment (start 109.28 137.61) (end 109.18 137.71) (width 0.2) (layer "F.Cu") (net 21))
 (segment (start 150.39 137.61) (end 109.28 137.61) (width 0.2) (layer "F.Cu") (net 21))
 (segment (start 150.39 90.09) (end 109.28 90.09) (width 0.2) (layer "B.Cu") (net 31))
 (segment (start 109.28 90.09) (end 109.18 90.19) (width 0.2) (layer "B.Cu") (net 31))
 (segment (start 150.39 70.29) (end 109.28 70.29) (width 0.2) (layer "B.Cu") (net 26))
 (segment (start 109.28 70.29) (end 109.18 70.39) (width 0.2) (layer "B.Cu") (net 26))
 (segment (start 150.39 117.81) (end 109.28 117.81) (width 0.2) (layer "F.Cu") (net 16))
 (segment (start 109.28 117.81) (end 109.18 117.91) (width 0.2) (layer "F.Cu") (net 16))
 (segment (start 109.28 125.73) (end 109.18 125.83) (width 0.2) (layer "F.Cu") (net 18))
 (segment (start 150.39 125.73) (end 109.28 125.73) (width 0.2) (layer "F.Cu") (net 18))
 (segment (start 109.28 82.16) (end 109.18 82.26) (width 0.2) (layer "F.Cu") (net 7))
 (segment (start 150.39 82.16) (end 109.28 82.16) (width 0.2) (layer "F.Cu") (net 7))
 (segment (start 109.28 94.05) (end 109.18 94.15) (width 0.2) (layer "B.Cu") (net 32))
 (segment (start 150.39 94.05) (end 109.28 94.05) (width 0.2) (layer "B.Cu") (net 32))
 (segment (start 150.39 137.61) (end 109.28 137.61) (width 0.2) (layer "B.Cu") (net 43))
 (segment (start 109.28 137.61) (end 109.18 137.71) (width 0.2) (layer "B.Cu") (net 43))
 (segment (start 109.28 94.05) (end 109.18 94.15) (width 0.2) (layer "F.Cu") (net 10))
 (segment (start 150.39 94.05) (end 109.28 94.05) (width 0.2) (layer "F.Cu") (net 10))
 (segment (start 109.28 90.09) (end 109.18 90.19) (width 0.2) (layer "F.Cu") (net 9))
 (segment (start 150.39 90.09) (end 109.28 90.09) (width 0.2) (layer "F.Cu") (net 9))
 (segment (start 150.39 113.85) (end 109.28 113.85) (width 0.2) (layer "B.Cu") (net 37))
 (segment (start 109.28 113.85) (end 109.18 113.95) (width 0.2) (layer "B.Cu") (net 37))
 (segment (start 109.28 129.69) (end 109.18 129.79) (width 0.2) (layer "B.Cu") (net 41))
 (segment (start 150.39 129.69) (end 109.28 129.69) (width 0.2) (layer "B.Cu") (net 41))
 (segment (start 109.28 66.33) (end 109.18 66.43) (width 0.2) (layer "B.Cu") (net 25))
 (segment (start 150.39 66.33) (end 109.28 66.33) (width 0.2) (layer "B.Cu") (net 25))
 (segment (start 109.28 66.33) (end 109.18 66.43) (width 0.2) (layer "F.Cu") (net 3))
 (segment (start 150.39 66.33) (end 109.28 66.33) (width 0.2) (layer "F.Cu") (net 3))
 (segment (start 109.28 101.97) (end 109.18 102.07) (width 0.2) (layer "F.Cu") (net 12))
 (segment (start 150.39 101.97) (end 109.28 101.97) (width 0.2) (layer "F.Cu") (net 12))
 (segment (start 109.28 109.89) (end 109.18 109.99) (width 0.2) (layer "B.Cu") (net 36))
 (segment (start 150.39 109.89) (end 109.28 109.89) (width 0.2) (layer "B.Cu") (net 36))
 (segment (start 150.39 86.13) (end 109.28 86.13) (width 0.2) (layer "B.Cu") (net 30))
 (segment (start 109.28 86.13) (end 109.18 86.23) (width 0.2) (layer "B.Cu") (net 30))
 (segment (start 150.29 141.66) (end 109.18 141.66) (width 0.2) (layer "B.Cu") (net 44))
 (segment (start 150.39 141.56) (end 150.29 141.66) (width 0.2) (layer "B.Cu") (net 44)))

